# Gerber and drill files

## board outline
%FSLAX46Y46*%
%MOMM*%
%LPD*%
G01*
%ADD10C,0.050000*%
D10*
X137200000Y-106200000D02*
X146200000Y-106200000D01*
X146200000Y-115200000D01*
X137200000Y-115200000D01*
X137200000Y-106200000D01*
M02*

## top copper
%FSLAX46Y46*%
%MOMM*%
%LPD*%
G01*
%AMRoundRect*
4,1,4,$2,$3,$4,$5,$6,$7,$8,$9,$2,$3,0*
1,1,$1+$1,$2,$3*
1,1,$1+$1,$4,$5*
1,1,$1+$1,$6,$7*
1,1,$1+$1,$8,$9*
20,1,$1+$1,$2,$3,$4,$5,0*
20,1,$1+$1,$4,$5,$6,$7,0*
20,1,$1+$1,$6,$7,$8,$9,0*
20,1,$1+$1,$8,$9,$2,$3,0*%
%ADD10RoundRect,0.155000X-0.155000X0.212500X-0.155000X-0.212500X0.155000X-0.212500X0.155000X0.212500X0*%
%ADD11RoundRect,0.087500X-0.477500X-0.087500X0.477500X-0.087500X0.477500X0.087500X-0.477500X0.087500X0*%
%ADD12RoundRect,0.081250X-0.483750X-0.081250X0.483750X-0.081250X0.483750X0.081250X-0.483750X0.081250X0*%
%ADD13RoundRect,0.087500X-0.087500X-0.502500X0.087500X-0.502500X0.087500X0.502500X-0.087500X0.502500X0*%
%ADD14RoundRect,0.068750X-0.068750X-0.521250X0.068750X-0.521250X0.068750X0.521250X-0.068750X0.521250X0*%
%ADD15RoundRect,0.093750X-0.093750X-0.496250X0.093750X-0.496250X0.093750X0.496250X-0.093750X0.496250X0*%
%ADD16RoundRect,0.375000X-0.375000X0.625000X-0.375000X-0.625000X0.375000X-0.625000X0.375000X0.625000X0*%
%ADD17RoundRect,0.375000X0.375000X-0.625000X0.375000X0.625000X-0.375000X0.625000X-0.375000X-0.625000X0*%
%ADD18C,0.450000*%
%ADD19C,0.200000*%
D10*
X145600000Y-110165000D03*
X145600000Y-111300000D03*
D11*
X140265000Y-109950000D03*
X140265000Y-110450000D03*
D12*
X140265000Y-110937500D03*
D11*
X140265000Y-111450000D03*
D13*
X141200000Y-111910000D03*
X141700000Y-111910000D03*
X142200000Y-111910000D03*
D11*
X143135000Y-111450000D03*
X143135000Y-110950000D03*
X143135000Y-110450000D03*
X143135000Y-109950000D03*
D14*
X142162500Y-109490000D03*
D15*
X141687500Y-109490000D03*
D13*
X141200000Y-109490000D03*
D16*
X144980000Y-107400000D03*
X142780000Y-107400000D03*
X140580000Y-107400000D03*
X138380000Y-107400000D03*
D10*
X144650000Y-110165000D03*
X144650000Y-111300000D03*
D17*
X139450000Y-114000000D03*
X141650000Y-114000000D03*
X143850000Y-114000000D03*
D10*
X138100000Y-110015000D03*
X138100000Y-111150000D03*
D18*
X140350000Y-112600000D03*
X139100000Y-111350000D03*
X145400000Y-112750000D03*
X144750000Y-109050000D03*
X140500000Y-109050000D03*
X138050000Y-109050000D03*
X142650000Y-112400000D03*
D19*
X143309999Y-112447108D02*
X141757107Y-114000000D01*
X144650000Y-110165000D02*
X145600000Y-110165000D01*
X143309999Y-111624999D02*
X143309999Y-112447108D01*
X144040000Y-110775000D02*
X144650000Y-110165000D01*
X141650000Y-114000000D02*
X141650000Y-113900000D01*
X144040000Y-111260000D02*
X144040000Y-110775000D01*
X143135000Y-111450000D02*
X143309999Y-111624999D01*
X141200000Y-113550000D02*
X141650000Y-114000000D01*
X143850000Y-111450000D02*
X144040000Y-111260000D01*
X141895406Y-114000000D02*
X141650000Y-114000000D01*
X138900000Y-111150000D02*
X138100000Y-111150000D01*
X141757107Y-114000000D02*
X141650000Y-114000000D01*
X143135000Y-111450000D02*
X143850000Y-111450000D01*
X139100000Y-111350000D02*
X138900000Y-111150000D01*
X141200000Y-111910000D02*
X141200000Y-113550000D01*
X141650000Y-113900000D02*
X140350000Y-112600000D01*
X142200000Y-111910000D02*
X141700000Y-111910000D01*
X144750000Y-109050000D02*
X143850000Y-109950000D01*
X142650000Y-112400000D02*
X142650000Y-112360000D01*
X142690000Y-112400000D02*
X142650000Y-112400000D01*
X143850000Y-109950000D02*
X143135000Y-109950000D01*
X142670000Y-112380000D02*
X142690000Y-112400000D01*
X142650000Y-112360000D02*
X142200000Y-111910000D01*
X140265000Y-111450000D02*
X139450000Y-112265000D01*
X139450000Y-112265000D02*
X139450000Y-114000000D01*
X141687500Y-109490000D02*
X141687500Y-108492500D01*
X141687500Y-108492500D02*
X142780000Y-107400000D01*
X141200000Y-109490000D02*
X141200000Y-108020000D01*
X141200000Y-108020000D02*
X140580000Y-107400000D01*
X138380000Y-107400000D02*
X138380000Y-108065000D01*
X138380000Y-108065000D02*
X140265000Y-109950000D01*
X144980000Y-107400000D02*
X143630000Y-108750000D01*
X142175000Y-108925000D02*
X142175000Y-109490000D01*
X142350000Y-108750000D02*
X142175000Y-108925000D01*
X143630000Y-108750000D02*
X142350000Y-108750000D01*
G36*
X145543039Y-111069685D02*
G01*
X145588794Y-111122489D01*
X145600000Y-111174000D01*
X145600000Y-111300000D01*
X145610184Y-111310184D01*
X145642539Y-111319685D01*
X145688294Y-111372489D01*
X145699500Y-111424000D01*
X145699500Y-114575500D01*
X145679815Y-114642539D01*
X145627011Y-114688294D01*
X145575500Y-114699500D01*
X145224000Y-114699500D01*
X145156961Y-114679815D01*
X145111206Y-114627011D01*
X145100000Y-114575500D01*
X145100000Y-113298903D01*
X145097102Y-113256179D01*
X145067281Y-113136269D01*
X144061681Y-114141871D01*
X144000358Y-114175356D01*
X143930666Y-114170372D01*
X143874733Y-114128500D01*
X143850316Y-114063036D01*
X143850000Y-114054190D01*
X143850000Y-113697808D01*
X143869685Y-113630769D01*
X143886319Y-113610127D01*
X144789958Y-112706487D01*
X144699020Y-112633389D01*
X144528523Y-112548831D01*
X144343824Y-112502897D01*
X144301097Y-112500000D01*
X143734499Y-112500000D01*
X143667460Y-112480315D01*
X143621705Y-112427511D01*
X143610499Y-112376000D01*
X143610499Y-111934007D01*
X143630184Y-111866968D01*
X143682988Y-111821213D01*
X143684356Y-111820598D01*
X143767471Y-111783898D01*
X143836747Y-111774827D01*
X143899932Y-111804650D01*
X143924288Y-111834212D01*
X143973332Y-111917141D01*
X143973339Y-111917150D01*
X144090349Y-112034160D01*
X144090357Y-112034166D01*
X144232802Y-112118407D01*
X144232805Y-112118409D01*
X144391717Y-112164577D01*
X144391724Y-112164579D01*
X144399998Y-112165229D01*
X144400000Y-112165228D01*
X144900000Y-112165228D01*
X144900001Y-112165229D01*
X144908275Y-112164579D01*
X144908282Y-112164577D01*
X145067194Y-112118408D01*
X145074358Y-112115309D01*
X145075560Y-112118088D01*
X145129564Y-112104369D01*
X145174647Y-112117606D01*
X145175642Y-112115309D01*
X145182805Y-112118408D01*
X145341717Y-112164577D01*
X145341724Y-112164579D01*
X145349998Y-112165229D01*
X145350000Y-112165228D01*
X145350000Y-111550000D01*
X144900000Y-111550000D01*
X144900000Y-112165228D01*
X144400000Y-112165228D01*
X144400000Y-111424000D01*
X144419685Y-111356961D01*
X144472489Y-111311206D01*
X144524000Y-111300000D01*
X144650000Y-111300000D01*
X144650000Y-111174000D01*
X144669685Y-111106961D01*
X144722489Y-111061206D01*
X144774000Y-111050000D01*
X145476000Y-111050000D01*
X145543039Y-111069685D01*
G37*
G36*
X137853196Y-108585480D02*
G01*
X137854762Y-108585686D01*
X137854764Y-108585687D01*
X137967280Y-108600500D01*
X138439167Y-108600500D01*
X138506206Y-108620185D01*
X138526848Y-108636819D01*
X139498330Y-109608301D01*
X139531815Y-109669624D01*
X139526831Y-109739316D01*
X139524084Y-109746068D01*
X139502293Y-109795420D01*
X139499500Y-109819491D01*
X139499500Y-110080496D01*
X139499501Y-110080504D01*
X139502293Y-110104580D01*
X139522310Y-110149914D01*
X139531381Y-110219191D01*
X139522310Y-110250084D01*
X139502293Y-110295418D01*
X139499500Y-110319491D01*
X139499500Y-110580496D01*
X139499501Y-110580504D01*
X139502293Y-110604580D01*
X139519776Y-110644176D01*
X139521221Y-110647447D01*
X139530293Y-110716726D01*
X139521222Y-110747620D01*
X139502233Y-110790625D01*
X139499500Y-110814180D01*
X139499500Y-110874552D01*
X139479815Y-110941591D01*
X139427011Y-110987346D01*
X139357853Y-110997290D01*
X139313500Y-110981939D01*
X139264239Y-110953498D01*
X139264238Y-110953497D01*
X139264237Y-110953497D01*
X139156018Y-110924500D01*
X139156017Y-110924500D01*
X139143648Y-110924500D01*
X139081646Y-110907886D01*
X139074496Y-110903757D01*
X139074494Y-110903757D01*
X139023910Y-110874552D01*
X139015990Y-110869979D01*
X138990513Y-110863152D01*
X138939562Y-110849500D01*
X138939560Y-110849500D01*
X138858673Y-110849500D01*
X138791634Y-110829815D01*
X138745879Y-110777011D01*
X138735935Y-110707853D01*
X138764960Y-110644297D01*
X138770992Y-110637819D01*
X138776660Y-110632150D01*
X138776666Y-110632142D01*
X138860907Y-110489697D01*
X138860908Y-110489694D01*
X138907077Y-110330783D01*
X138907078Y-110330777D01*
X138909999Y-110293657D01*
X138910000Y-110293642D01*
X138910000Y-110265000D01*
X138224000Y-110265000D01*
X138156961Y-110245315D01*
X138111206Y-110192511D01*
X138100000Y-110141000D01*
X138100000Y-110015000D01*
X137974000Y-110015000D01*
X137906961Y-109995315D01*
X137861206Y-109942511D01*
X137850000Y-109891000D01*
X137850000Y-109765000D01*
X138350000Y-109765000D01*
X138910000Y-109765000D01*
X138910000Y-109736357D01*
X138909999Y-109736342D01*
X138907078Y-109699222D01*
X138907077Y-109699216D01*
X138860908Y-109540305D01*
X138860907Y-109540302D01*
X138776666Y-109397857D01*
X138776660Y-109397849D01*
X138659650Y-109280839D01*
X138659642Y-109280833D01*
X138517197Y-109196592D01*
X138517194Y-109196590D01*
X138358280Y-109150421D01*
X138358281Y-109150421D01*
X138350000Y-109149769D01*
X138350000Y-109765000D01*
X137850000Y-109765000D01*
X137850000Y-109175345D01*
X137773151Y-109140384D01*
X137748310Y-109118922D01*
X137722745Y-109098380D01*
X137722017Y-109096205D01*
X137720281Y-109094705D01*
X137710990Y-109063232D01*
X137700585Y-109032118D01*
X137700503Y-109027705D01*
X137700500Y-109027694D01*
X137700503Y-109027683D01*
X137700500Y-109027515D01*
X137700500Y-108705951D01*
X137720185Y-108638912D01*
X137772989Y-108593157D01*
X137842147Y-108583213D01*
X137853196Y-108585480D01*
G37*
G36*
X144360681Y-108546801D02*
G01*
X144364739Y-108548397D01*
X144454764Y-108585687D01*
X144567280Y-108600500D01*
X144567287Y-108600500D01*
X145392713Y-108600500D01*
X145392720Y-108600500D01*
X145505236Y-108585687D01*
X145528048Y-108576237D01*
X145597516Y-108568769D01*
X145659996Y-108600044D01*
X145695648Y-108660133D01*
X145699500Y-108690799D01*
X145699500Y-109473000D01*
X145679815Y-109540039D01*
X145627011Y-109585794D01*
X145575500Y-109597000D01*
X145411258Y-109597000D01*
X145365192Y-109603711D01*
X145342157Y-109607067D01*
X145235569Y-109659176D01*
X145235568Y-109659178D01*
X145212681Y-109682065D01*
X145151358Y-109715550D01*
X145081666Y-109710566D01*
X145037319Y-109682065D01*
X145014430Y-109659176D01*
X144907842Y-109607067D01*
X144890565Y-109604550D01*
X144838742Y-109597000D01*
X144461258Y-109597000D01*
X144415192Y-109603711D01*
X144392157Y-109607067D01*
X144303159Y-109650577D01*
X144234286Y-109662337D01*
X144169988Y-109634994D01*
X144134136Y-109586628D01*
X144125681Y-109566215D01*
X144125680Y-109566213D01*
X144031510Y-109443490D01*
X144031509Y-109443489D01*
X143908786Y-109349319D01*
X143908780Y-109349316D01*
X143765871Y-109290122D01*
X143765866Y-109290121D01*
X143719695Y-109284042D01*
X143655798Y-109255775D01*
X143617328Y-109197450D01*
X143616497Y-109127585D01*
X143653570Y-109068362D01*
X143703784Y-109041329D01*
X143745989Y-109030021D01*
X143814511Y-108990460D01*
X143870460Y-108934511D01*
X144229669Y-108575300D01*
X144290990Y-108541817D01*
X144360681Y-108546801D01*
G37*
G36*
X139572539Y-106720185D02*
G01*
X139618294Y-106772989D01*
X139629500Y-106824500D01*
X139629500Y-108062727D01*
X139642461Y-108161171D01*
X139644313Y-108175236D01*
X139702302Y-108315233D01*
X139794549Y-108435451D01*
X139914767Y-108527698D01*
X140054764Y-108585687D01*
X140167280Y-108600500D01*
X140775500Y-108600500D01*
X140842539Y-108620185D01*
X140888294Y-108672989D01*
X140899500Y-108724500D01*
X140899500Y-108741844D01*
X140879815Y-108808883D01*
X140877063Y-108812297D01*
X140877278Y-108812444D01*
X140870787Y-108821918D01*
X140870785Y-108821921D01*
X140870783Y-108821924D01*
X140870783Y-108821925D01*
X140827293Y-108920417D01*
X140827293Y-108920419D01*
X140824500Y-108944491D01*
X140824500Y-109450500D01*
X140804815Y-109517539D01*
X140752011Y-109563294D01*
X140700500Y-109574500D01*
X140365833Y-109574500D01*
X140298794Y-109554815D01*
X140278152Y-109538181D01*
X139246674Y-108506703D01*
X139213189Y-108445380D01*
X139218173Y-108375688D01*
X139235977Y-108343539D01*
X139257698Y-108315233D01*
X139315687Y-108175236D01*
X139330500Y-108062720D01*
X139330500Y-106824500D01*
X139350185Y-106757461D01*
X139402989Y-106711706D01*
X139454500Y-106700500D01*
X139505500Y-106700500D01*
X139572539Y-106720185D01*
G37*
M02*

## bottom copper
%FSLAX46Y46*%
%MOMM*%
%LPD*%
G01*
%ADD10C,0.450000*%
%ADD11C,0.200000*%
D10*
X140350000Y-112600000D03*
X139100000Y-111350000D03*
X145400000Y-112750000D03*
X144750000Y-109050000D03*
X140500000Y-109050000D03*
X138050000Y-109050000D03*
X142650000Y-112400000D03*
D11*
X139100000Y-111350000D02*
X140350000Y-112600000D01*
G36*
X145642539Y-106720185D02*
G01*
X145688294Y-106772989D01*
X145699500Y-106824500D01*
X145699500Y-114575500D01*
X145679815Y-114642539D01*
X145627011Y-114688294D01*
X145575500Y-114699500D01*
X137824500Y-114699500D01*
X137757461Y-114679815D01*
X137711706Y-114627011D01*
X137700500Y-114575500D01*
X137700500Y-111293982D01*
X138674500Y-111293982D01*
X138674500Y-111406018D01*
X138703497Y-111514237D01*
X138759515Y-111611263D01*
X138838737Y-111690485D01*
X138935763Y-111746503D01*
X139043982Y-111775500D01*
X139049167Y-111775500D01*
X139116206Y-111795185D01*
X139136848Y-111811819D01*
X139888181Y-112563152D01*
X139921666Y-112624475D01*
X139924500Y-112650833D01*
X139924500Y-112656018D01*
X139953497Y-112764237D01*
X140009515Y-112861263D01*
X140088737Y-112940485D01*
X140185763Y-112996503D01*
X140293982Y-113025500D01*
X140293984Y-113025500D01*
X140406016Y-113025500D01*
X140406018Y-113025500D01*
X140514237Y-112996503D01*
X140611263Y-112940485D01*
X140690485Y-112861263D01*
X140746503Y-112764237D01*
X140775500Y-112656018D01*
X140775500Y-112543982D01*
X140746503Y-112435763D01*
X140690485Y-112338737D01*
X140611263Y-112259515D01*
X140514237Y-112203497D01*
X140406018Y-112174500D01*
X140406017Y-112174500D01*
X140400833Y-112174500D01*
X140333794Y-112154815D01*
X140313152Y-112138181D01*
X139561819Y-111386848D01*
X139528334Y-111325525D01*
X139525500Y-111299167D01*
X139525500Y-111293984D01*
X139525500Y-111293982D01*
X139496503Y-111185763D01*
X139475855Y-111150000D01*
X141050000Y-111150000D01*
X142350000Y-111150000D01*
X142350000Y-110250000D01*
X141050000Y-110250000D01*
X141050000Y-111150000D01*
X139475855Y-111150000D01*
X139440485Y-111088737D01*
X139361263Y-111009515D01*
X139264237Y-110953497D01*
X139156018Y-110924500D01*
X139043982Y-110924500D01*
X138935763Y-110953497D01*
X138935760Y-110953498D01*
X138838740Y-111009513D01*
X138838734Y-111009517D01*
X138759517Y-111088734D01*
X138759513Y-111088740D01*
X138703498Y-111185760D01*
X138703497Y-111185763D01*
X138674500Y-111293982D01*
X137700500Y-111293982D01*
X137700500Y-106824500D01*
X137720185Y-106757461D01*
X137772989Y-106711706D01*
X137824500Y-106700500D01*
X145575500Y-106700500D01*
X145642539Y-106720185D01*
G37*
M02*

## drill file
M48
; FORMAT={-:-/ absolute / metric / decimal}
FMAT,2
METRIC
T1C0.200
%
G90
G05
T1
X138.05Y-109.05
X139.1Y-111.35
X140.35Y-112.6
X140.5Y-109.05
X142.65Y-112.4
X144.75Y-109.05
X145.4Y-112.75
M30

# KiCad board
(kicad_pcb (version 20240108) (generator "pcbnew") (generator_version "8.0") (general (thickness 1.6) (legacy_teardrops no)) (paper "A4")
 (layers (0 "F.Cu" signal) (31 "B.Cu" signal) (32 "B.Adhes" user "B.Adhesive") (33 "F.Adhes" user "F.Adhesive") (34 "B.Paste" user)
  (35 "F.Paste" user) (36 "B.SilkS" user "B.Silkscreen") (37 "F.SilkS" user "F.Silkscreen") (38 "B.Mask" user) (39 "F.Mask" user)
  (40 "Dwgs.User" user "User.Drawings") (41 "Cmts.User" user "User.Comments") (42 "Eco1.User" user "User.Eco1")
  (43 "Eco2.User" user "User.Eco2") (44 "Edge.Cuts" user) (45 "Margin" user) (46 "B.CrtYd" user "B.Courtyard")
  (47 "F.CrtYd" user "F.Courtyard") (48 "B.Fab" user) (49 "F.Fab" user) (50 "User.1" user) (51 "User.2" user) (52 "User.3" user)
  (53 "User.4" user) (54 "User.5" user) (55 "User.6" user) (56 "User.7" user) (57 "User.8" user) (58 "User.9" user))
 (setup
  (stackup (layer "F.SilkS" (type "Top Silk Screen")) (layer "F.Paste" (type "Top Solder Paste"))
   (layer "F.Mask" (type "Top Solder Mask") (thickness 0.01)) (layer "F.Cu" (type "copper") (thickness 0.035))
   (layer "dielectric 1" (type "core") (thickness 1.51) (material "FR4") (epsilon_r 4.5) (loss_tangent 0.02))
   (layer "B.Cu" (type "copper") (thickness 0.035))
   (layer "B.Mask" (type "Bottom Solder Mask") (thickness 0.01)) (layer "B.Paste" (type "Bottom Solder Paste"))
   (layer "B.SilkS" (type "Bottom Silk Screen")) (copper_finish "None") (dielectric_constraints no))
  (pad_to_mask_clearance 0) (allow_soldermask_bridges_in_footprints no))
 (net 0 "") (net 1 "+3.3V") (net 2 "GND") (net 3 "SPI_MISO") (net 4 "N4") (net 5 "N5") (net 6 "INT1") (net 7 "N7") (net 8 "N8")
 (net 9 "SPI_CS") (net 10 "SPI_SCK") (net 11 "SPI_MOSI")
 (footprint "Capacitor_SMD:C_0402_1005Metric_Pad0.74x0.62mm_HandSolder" (layer "F.Cu") (at 145.6 110.7325 -90)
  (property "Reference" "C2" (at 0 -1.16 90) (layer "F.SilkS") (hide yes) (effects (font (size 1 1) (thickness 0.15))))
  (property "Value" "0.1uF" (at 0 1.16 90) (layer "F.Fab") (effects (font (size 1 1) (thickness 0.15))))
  (pad "1" smd roundrect (at -0.5675 0 270) (size 0.735 0.62) (layers "F.Cu" "F.Paste" "F.Mask") (roundrect_rratio 0.25) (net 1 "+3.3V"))
  (pad "2" smd roundrect (at 0.5675 0 270) (size 0.735 0.62) (layers "F.Cu" "F.Paste" "F.Mask") (roundrect_rratio 0.25) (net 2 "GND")))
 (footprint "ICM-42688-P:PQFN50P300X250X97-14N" (layer "F.Cu") (at 141.7 110.7)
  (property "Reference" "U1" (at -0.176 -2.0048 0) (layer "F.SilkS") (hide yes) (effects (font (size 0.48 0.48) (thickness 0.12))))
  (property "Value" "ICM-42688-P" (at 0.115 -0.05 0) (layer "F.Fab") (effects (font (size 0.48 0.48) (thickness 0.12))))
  (pad "1" smd roundrect (at -1.435 -0.75) (size 1.13 0.35) (layers "F.Cu" "F.Paste") (roundrect_rratio 0.25) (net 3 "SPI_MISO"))
  (pad "2" smd roundrect (at -1.435 -0.25) (size 1.13 0.35) (layers "F.Cu" "F.Paste") (roundrect_rratio 0.25) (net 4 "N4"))
  (pad "3" smd roundrect (at -1.435 0.2375) (size 1.13 0.325) (layers "F.Cu" "F.Paste") (roundrect_rratio 0.25) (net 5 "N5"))
  (pad "4" smd roundrect (at -1.435 0.75) (size 1.13 0.35) (layers "F.Cu" "F.Paste") (roundrect_rratio 0.25) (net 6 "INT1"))
  (pad "5" smd roundrect (at -0.5 1.21) (size 0.35 1.18) (layers "F.Cu" "F.Paste") (roundrect_rratio 0.25) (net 1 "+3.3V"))
  (pad "6" smd roundrect (at 0 1.21) (size 0.35 1.18) (layers "F.Cu" "F.Paste") (roundrect_rratio 0.25) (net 2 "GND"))
  (pad "7" smd roundrect (at 0.5 1.21) (size 0.35 1.18) (layers "F.Cu" "F.Paste") (roundrect_rratio 0.25) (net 2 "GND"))
  (pad "8" smd roundrect (at 1.435 0.75) (size 1.13 0.35) (layers "F.Cu" "F.Paste") (roundrect_rratio 0.25) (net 1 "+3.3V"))
  (pad "9" smd roundrect (at 1.435 0.25) (size 1.13 0.35) (layers "F.Cu" "F.Paste") (roundrect_rratio 0.25) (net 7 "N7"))
  (pad "10" smd roundrect (at 1.435 -0.25) (size 1.13 0.35) (layers "F.Cu" "F.Paste") (roundrect_rratio 0.25) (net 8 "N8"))
  (pad "11" smd roundrect (at 1.435 -0.75) (size 1.13 0.35) (layers "F.Cu" "F.Paste") (roundrect_rratio 0.25) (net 2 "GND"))
  (pad "12" smd roundrect (at 0.4625 -1.21) (size 0.275 1.18) (layers "F.Cu" "F.Paste") (roundrect_rratio 0.25) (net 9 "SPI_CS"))
  (pad "13" smd roundrect (at -0.0125 -1.21) (size 0.375 1.18) (layers "F.Cu" "F.Paste") (roundrect_rratio 0.25) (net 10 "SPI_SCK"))
  (pad "14" smd roundrect (at -0.5 -1.21) (size 0.35 1.18) (layers "F.Cu" "F.Paste") (roundrect_rratio 0.25) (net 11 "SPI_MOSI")))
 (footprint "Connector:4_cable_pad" (layer "F.Cu") (at 145.78 106.2 180)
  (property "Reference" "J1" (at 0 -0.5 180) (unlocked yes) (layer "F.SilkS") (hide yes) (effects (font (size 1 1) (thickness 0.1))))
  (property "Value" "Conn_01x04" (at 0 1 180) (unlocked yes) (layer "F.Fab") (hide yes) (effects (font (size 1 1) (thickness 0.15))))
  (pad "1" smd roundrect (at 0.8 -1.2 270) (size 2 1.5) (layers "F.Cu" "F.Paste" "F.Mask") (roundrect_rratio 0.25) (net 9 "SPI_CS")
   (thermal_bridge_angle 45))
  (pad "2" smd roundrect (at 3 -1.2 270) (size 2 1.5) (layers "F.Cu" "F.Paste" "F.Mask") (roundrect_rratio 0.25) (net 10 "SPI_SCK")
   (thermal_bridge_angle 45))
  (pad "3" smd roundrect (at 5.2 -1.2 270) (size 2 1.5) (layers "F.Cu" "F.Paste" "F.Mask") (roundrect_rratio 0.25) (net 11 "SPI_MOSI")
   (thermal_bridge_angle 45))
  (pad "4" smd roundrect (at 7.4 -1.2 270) (size 2 1.5) (layers "F.Cu" "F.Paste" "F.Mask") (roundrect_rratio 0.25) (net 3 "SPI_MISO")
   (thermal_bridge_angle 45)))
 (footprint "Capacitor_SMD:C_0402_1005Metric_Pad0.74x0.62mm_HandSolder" (layer "F.Cu") (at 144.65 110.7325 -90)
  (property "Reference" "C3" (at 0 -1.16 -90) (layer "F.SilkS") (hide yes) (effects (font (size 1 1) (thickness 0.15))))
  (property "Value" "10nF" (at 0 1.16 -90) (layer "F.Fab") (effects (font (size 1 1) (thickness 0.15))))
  (pad "1" smd roundrect (at -0.5675 0 270) (size 0.735 0.62) (layers "F.Cu" "F.Paste" "F.Mask") (roundrect_rratio 0.25) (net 1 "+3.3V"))
  (pad "2" smd roundrect (at 0.5675 0 270) (size 0.735 0.62) (layers "F.Cu" "F.Paste" "F.Mask") (roundrect_rratio 0.25) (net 2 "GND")))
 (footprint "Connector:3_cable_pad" (layer "F.Cu") (at 138.65 115.2)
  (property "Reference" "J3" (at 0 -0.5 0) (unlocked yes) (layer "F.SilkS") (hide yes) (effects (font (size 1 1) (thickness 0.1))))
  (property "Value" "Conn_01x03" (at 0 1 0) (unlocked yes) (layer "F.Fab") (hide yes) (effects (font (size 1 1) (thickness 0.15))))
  (pad "1" smd roundrect (at 0.8 -1.2 90) (size 2 1.5) (layers "F.Cu" "F.Paste" "F.Mask") (roundrect_rratio 0.25) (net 6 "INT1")
   (thermal_bridge_angle 45))
  (pad "2" smd roundrect (at 3 -1.2 90) (size 2 1.5) (layers "F.Cu" "F.Paste" "F.Mask") (roundrect_rratio 0.25) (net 1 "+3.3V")
   (thermal_bridge_angle 45))
  (pad "3" smd roundrect (at 5.2 -1.2 90) (size 2 1.5) (layers "F.Cu" "F.Paste" "F.Mask") (roundrect_rratio 0.25) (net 2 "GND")
   (thermal_bridge_angle 45)))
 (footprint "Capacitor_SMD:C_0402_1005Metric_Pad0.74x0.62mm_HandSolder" (layer "F.Cu") (at 138.1 110.5825 -90)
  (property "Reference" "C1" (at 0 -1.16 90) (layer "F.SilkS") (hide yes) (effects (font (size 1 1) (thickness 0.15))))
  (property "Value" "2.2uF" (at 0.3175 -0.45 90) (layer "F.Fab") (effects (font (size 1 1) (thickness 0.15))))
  (pad "1" smd roundrect (at -0.5675 0 270) (size 0.735 0.62) (layers "F.Cu" "F.Paste" "F.Mask") (roundrect_rratio 0.25) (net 2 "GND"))
  (pad "2" smd roundrect (at 0.5675 0 270) (size 0.735 0.62) (layers "F.Cu" "F.Paste" "F.Mask") (roundrect_rratio 0.25) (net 1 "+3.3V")))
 (gr_rect (start 137.2 106.2) (end 146.2 115.2) (stroke (width 0.05) (type default)) (fill none) (layer "Edge.Cuts"))
 (segment (start 143.309999 112.447108) (end 141.757107 114) (width 0.2) (layer "F.Cu") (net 1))
 (segment (start 144.65 110.165) (end 145.6 110.165) (width 0.2) (layer "F.Cu") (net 1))
 (segment (start 143.309999 111.624999) (end 143.309999 112.447108) (width 0.2) (layer "F.Cu") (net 1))
 (segment (start 144.04 110.775) (end 144.65 110.165) (width 0.2) (layer "F.Cu") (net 1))
 (segment (start 141.65 114) (end 141.65 113.9) (width 0.2) (layer "F.Cu") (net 1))
 (segment (start 144.04 111.26) (end 144.04 110.775) (width 0.2) (layer "F.Cu") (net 1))
 (segment (start 143.135 111.45) (end 143.309999 111.624999) (width 0.2) (layer "F.Cu") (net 1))
 (segment (start 141.2 113.55) (end 141.65 114) (width 0.2) (layer "F.Cu") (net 1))
 (segment (start 143.85 111.45) (end 144.04 111.26) (width 0.2) (layer "F.Cu") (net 1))
 (segment (start 141.895406 114) (end 141.65 114) (width 0.2) (layer "F.Cu") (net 1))
 (segment (start 138.9 111.15) (end 138.1 111.15) (width 0.2) (layer "F.Cu") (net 1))
 (segment (start 141.757107 114) (end 141.65 114) (width 0.2) (layer "F.Cu") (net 1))
 (segment (start 143.135 111.45) (end 143.85 111.45) (width 0.2) (layer "F.Cu") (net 1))
 (segment (start 139.1 111.35) (end 138.9 111.15) (width 0.2) (layer "F.Cu") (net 1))
 (segment (start 141.2 111.91) (end 141.2 113.55) (width 0.2) (layer "F.Cu") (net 1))
 (segment (start 141.65 113.9) (end 140.35 112.6) (width 0.2) (layer "F.Cu") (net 1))
 (via (at 140.35 112.6) (size 0.45) (drill 0.2) (layers "F.Cu" "B.Cu") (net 1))
 (via (at 139.1 111.35) (size 0.45) (drill 0.2) (layers "F.Cu" "B.Cu") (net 1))
 (segment (start 139.1 111.35) (end 140.35 112.6) (width 0.2) (layer "B.Cu") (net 1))
 (segment (start 142.2 111.91) (end 141.7 111.91) (width 0.2) (layer "F.Cu") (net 2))
 (segment (start 144.75 109.05) (end 143.85 109.95) (width 0.2) (layer "F.Cu") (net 2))
 (segment (start 142.65 112.4) (end 142.65 112.36) (width 0.2) (layer "F.Cu") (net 2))
 (segment (start 142.69 112.4) (end 142.65 112.4) (width 0.2) (layer "F.Cu") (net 2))
 (segment (start 143.85 109.95) (end 143.135 109.95) (width 0.2) (layer "F.Cu") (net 2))
 (segment (start 142.67 112.38) (end 142.69 112.4) (width 0.2) (layer "F.Cu") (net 2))
 (segment (start 142.65 112.36) (end 142.2 111.91) (width 0.2) (layer "F.Cu") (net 2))
 (via (at 145.4 112.75) (size 0.45) (drill 0.2) (layers "F.Cu" "B.Cu") (free yes) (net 2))
 (via (at 144.75 109.05) (size 0.45) (drill 0.2) (layers "F.Cu" "B.Cu") (free yes) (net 2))
 (via (at 140.5 109.05) (size 0.45) (drill 0.2) (layers "F.Cu" "B.Cu") (free yes) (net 2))
 (via (at 138.05 109.05) (size 0.45) (drill 0.2) (layers "F.Cu" "B.Cu") (free yes) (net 2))
 (via (at 142.65 112.4) (size 0.45) (drill 0.2) (layers "F.Cu" "B.Cu") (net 2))
 (segment (start 140.265 111.45) (end 139.45 112.265) (width 0.2) (layer "F.Cu") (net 6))
 (segment (start 139.45 112.265) (end 139.45 114) (width 0.2) (layer "F.Cu") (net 6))
 (segment (start 141.6875 109.49) (end 141.6875 108.4925) (width 0.2) (layer "F.Cu") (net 10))
 (segment (start 141.6875 108.4925) (end 142.78 107.4) (width 0.2) (layer "F.Cu") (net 10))
 (segment (start 141.2 109.49) (end 141.2 108.02) (width 0.2) (layer "F.Cu") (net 11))
 (segment (start 141.2 108.02) (end 140.58 107.4) (width 0.2) (layer "F.Cu") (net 11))
 (segment (start 138.38 107.4) (end 138.38 108.065) (width 0.2) (layer "F.Cu") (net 3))
 (segment (start 138.38 108.065) (end 140.265 109.95) (width 0.2) (layer "F.Cu") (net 3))
 (segment (start 144.98 107.4) (end 143.63 108.75) (width 0.2) (layer "F.Cu") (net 9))
 (segment (start 142.175 108.925) (end 142.175 109.49) (width 0.2) (layer "F.Cu") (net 9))
 (segment (start 142.35 108.75) (end 142.175 108.925) (width 0.2) (layer "F.Cu") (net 9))
 (segment (start 143.63 108.75) (end 142.35 108.75) (width 0.2) (layer "F.Cu") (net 9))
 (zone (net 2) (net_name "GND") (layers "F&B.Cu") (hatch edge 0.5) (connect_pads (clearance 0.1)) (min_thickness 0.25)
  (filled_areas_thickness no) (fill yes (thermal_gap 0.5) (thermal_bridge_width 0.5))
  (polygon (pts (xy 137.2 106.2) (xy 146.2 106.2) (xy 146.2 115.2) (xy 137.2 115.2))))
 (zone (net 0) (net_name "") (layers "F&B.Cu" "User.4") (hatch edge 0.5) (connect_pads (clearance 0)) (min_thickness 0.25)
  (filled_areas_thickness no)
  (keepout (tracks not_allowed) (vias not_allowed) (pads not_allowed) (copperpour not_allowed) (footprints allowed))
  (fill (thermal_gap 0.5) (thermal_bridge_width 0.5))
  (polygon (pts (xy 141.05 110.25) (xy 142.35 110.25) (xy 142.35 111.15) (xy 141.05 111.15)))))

